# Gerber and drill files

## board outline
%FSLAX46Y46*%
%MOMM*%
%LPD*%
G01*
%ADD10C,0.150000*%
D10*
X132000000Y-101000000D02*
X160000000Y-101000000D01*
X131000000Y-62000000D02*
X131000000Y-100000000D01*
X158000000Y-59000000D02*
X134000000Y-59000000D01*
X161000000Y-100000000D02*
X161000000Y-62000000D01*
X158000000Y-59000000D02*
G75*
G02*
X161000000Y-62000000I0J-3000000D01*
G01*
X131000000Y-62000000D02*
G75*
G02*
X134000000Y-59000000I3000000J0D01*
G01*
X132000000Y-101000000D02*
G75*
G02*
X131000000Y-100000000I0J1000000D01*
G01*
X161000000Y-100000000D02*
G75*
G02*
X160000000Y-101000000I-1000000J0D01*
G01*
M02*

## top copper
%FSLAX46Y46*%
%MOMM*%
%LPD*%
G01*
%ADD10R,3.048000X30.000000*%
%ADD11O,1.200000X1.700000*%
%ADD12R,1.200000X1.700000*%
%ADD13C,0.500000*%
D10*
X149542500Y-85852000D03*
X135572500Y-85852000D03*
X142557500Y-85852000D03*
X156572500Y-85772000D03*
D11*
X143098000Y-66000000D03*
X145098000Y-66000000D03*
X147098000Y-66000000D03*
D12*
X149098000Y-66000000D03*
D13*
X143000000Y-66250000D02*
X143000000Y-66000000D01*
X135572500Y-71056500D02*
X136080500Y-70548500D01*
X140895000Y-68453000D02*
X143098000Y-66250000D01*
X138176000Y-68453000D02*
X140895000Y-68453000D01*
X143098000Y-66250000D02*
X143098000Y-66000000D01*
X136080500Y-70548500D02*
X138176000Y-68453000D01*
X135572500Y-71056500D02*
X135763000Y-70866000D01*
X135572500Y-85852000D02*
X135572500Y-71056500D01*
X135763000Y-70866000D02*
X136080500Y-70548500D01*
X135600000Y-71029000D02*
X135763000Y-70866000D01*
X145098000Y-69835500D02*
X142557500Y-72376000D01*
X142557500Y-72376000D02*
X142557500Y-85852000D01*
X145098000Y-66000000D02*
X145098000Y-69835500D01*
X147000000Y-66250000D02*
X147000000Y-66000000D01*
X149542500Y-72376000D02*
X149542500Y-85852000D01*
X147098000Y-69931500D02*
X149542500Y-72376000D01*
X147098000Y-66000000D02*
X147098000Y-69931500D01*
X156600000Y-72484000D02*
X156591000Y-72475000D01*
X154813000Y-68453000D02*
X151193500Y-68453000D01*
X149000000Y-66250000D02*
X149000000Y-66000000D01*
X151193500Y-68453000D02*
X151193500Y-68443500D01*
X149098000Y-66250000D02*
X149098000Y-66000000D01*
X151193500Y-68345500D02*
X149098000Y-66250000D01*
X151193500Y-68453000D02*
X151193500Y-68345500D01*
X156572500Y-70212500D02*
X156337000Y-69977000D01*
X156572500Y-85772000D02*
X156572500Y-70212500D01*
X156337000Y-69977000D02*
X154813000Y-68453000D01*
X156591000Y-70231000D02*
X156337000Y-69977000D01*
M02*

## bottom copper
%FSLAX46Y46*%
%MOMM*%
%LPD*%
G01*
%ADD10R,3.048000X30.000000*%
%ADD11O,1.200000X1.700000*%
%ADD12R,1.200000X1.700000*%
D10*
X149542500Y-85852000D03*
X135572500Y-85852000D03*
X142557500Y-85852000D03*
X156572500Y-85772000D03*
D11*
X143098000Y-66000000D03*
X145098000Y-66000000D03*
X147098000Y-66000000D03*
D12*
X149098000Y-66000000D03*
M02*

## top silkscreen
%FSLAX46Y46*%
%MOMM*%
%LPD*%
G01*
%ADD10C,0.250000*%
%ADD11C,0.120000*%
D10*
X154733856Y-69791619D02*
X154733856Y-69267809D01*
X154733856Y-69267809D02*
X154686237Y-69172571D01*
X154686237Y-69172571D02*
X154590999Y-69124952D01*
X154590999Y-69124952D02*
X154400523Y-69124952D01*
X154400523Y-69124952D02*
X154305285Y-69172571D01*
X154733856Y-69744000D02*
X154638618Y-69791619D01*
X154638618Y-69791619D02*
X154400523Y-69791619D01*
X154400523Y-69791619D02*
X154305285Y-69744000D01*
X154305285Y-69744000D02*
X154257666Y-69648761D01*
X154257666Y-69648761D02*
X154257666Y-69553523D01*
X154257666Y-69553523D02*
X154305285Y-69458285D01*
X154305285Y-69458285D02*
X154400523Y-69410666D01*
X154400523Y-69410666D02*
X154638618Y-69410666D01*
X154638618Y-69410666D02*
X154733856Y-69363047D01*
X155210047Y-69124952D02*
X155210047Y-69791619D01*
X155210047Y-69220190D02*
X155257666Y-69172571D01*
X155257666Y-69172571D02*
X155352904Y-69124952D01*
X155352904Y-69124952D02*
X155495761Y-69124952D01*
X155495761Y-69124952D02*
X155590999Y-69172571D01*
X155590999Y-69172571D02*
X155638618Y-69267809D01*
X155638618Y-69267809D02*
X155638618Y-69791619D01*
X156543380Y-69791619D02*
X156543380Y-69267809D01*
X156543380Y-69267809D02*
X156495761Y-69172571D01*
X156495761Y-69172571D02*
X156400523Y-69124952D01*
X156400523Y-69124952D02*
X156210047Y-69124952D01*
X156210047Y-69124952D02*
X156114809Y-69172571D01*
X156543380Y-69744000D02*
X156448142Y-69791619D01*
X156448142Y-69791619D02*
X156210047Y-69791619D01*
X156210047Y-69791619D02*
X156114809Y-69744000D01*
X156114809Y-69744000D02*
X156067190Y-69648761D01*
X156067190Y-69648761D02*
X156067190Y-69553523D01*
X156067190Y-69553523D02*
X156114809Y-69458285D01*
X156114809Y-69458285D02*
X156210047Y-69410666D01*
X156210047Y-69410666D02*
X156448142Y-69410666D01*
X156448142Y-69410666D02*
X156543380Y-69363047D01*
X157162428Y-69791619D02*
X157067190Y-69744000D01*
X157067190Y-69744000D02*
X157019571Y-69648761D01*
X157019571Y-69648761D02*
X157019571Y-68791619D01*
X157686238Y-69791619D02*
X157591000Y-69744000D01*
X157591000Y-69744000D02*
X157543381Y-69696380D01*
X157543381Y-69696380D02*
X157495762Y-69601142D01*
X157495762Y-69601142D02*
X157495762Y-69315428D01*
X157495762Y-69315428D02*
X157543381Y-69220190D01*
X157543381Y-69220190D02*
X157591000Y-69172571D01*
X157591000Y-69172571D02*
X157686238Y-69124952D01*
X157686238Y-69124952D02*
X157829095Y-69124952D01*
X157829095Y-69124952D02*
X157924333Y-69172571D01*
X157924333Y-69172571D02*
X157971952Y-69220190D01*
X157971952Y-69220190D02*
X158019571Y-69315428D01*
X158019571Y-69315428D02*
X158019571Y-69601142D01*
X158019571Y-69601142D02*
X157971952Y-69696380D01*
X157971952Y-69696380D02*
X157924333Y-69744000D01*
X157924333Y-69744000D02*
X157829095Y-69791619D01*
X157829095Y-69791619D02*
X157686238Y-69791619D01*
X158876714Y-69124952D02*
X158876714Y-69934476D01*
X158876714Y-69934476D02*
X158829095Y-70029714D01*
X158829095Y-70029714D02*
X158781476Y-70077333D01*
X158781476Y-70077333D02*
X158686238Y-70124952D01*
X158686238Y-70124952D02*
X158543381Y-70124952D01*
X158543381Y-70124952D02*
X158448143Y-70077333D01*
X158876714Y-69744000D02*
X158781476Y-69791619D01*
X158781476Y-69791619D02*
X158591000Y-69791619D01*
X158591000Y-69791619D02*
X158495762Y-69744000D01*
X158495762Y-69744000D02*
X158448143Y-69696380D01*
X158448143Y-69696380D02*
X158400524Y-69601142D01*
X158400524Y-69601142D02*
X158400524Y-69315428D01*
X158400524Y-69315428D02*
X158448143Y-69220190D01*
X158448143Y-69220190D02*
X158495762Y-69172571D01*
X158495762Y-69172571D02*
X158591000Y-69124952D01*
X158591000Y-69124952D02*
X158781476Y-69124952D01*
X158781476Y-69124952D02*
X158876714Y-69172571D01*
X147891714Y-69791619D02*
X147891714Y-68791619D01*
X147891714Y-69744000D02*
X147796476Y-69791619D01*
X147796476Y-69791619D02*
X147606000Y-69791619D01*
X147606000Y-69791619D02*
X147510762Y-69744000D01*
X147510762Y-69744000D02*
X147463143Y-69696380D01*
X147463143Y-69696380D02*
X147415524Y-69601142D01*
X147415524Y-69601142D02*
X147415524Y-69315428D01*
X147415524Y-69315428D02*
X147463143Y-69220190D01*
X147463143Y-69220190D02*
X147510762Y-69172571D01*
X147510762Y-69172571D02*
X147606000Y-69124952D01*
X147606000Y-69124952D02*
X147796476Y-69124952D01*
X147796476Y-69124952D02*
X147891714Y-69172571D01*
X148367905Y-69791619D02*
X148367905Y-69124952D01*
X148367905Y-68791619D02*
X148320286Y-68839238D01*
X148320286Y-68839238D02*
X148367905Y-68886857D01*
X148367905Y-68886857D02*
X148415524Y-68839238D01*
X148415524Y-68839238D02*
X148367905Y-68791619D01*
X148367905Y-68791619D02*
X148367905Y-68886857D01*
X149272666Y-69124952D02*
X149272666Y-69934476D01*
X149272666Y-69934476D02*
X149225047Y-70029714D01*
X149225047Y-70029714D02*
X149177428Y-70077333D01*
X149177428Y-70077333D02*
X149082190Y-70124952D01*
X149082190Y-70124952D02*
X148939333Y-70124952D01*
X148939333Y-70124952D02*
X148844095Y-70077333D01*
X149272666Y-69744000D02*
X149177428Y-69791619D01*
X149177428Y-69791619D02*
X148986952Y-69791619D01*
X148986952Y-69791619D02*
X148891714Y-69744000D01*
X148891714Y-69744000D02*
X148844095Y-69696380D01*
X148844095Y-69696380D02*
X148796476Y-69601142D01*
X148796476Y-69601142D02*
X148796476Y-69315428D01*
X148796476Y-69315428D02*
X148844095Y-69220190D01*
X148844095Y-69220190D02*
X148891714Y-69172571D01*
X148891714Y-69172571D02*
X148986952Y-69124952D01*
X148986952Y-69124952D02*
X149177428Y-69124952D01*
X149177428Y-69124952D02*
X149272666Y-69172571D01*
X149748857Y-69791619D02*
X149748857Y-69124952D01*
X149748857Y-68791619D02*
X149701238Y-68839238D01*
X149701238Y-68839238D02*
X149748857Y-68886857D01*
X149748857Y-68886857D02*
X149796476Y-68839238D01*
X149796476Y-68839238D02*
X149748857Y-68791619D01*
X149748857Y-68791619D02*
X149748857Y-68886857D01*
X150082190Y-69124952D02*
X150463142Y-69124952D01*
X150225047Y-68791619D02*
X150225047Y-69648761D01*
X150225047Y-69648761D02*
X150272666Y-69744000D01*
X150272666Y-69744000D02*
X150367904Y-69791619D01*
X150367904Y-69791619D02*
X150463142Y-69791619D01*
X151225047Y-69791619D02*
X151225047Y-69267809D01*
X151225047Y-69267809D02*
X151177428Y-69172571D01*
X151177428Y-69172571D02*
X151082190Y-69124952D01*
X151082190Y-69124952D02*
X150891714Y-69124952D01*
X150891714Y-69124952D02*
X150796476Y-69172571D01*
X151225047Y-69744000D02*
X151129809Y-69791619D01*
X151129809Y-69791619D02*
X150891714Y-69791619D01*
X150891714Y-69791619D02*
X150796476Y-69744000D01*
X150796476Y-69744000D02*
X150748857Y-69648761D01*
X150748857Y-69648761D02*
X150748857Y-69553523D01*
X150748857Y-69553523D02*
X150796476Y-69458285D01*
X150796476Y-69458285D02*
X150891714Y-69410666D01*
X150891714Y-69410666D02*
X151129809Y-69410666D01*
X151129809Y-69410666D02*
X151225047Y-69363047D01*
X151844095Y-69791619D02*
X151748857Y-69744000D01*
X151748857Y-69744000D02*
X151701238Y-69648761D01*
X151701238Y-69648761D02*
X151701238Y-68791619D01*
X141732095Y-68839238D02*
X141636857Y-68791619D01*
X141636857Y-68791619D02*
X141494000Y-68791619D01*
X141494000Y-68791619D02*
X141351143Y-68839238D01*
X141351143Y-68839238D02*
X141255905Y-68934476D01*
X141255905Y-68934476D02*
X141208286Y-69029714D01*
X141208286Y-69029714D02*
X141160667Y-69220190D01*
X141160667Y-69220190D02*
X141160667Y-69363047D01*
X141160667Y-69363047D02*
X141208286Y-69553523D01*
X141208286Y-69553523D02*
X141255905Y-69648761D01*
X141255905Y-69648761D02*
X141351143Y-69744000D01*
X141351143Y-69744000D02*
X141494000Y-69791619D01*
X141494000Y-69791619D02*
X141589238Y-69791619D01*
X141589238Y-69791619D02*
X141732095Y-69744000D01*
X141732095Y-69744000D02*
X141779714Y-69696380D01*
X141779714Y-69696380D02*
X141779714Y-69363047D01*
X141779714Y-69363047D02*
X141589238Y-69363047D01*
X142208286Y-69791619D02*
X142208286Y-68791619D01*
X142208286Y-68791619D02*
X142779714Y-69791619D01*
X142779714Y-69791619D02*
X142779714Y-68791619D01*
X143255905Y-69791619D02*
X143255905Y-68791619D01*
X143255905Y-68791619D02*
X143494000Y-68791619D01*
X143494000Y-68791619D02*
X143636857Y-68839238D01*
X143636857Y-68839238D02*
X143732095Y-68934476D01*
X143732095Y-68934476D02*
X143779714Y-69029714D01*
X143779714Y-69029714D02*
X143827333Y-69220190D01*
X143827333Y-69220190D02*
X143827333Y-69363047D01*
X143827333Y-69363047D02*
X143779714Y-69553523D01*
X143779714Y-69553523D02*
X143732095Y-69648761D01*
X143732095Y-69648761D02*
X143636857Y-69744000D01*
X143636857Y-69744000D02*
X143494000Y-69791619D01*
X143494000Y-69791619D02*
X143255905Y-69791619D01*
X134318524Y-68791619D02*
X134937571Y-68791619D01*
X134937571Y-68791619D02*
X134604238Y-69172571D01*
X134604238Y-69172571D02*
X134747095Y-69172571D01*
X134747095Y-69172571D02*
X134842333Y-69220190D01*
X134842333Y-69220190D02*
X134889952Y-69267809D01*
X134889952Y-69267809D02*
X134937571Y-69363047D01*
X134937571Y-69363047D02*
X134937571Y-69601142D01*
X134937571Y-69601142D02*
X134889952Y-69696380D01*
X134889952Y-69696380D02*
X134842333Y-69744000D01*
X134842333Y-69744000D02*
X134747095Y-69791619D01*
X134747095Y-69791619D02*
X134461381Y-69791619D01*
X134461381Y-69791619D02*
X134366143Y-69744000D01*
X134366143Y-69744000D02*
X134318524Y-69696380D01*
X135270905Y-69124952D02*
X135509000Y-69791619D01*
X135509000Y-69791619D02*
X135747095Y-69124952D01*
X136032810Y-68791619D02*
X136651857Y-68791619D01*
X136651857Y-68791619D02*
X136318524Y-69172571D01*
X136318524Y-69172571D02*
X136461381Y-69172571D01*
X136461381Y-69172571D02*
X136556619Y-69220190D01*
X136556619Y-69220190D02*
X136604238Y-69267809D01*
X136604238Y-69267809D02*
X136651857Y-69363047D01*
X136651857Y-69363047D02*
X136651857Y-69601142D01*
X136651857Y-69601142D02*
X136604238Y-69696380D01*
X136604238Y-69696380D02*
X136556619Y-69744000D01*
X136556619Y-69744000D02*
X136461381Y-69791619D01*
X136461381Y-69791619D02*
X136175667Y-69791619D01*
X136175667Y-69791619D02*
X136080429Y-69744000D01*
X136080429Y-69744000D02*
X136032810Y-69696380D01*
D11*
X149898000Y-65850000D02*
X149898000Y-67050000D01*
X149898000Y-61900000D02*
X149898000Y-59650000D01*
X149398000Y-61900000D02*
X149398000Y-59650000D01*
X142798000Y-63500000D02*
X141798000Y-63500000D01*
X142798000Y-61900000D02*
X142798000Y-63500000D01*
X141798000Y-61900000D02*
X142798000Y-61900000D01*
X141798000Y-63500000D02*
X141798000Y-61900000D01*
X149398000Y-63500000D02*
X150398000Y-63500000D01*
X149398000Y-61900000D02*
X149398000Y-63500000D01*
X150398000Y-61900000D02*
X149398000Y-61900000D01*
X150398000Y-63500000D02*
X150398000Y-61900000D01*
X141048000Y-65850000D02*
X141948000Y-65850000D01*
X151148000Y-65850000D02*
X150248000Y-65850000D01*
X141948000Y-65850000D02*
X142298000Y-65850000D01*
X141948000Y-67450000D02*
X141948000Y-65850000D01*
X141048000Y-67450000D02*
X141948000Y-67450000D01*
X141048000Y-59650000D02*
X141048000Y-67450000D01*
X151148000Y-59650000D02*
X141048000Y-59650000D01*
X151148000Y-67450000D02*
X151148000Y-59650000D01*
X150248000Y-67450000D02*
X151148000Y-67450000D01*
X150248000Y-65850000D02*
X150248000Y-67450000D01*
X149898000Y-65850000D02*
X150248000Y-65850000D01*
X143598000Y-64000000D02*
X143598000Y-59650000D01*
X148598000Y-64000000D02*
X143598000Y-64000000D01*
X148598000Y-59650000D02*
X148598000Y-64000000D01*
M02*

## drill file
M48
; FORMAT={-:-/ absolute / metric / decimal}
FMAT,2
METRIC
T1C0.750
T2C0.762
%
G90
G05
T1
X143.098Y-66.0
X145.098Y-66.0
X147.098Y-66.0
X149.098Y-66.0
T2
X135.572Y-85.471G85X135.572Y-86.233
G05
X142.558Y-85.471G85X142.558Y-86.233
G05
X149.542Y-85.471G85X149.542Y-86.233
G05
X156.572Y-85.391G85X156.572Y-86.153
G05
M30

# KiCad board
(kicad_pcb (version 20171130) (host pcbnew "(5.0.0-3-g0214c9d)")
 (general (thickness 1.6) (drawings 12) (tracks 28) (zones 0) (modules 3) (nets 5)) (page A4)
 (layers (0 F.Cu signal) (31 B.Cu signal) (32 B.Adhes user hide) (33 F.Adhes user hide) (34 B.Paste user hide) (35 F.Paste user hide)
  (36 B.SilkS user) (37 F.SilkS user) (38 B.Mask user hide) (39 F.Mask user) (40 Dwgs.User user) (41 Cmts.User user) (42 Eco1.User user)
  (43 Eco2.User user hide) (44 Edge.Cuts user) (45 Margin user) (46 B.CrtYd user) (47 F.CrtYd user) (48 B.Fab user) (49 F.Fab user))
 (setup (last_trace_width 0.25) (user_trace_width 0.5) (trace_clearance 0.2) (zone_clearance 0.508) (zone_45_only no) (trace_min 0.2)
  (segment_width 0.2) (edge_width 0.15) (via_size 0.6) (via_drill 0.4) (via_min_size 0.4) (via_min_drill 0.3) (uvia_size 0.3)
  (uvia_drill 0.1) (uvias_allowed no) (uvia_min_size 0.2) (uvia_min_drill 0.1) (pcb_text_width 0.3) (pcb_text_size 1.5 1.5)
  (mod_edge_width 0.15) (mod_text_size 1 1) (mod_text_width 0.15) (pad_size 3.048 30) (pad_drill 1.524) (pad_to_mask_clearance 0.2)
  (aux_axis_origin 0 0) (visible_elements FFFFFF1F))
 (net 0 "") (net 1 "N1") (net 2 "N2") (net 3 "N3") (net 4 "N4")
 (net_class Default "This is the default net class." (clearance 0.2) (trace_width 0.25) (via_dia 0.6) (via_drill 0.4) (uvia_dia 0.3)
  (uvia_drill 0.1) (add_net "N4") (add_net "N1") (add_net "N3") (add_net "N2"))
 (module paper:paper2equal (layer B.Cu) (at 145.7325 70.612)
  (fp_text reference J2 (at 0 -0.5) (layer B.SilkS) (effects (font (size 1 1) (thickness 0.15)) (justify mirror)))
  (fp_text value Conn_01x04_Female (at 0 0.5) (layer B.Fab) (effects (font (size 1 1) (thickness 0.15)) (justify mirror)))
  (pad 3 thru_hole rect (at 3.81 15.24) (size 3.048 30) (drill oval 0.762 1.524) (layers *.Cu *.Mask) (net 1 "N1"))
  (pad 1 thru_hole rect (at -10.16 15.24) (size 3.048 30) (drill oval 0.762 1.524) (layers *.Cu *.Mask) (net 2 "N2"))
  (pad 2 thru_hole rect (at -3.175 15.24) (size 3.048 30) (drill oval 0.762 1.524) (layers *.Cu *.Mask) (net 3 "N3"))
  (pad 4 thru_hole rect (at 10.84 15.16) (size 3.048 30) (drill oval 0.762 1.524) (layers *.Cu *.Mask) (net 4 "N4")))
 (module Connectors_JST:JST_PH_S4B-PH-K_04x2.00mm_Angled (layer F.Cu) (at 149.098 66 180)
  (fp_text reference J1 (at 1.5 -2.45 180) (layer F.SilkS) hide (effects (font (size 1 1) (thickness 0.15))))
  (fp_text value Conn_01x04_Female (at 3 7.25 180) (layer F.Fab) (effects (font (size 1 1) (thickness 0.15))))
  (fp_line (start -0.8 0.15) (end -0.8 -1.05) (layer F.SilkS) (width 0.12))
  (fp_line (start -0.8 4.1) (end -0.8 6.35) (layer F.SilkS) (width 0.12))
  (fp_line (start -0.3 4.1) (end -0.3 6.35) (layer F.SilkS) (width 0.12))
  (fp_line (start 6.3 2.5) (end 7.3 2.5) (layer F.SilkS) (width 0.12))
  (fp_line (start 6.3 4.1) (end 6.3 2.5) (layer F.SilkS) (width 0.12))
  (fp_line (start 7.3 4.1) (end 6.3 4.1) (layer F.SilkS) (width 0.12))
  (fp_line (start 7.3 2.5) (end 7.3 4.1) (layer F.SilkS) (width 0.12))
  (fp_line (start -0.3 2.5) (end -1.3 2.5) (layer F.SilkS) (width 0.12))
  (fp_line (start -0.3 4.1) (end -0.3 2.5) (layer F.SilkS) (width 0.12))
  (fp_line (start -1.3 4.1) (end -0.3 4.1) (layer F.SilkS) (width 0.12))
  (fp_line (start -1.3 2.5) (end -1.3 4.1) (layer F.SilkS) (width 0.12))
  (fp_line (start 8.05 0.15) (end 7.15 0.15) (layer F.SilkS) (width 0.12))
  (fp_line (start -2.05 0.15) (end -1.15 0.15) (layer F.SilkS) (width 0.12))
  (fp_line (start 7.15 0.15) (end 6.8 0.15) (layer F.SilkS) (width 0.12))
  (fp_line (start 7.15 -1.45) (end 7.15 0.15) (layer F.SilkS) (width 0.12))
  (fp_line (start 8.05 -1.45) (end 7.15 -1.45) (layer F.SilkS) (width 0.12))
  (fp_line (start 8.05 6.35) (end 8.05 -1.45) (layer F.SilkS) (width 0.12))
  (fp_line (start -2.05 6.35) (end 8.05 6.35) (layer F.SilkS) (width 0.12))
  (fp_line (start -2.05 -1.45) (end -2.05 6.35) (layer F.SilkS) (width 0.12))
  (fp_line (start -1.15 -1.45) (end -2.05 -1.45) (layer F.SilkS) (width 0.12))
  (fp_line (start -1.15 0.15) (end -1.15 -1.45) (layer F.SilkS) (width 0.12))
  (fp_line (start -0.8 0.15) (end -1.15 0.15) (layer F.SilkS) (width 0.12))
  (fp_line (start 5.5 2) (end 5.5 6.35) (layer F.SilkS) (width 0.12))
  (fp_line (start 0.5 2) (end 5.5 2) (layer F.SilkS) (width 0.12))
  (fp_line (start 0.5 6.35) (end 0.5 2) (layer F.SilkS) (width 0.12))
  (pad 4 thru_hole oval (at 6 0 180) (size 1.2 1.7) (drill 0.75) (layers *.Cu *.Mask) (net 2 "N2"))
  (pad 3 thru_hole oval (at 4 0 180) (size 1.2 1.7) (drill 0.75) (layers *.Cu *.Mask) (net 3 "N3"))
  (pad 2 thru_hole oval (at 2 0 180) (size 1.2 1.7) (drill 0.75) (layers *.Cu *.Mask) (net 1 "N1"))
  (pad 1 thru_hole rect (at 0 0 180) (size 1.2 1.7) (drill 0.75) (layers *.Cu *.Mask) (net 4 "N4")))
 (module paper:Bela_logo (layer B.Cu) (at 155.067 64.897 135)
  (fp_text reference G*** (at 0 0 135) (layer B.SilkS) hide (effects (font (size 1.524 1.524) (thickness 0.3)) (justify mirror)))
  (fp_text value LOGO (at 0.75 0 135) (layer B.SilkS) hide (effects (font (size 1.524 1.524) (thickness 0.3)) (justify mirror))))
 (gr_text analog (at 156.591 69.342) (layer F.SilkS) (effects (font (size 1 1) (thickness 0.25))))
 (gr_line (start 132 101) (end 160 101) (angle 90) (layer Edge.Cuts) (width 0.15))
 (gr_line (start 131 62) (end 131 100) (angle 90) (layer Edge.Cuts) (width 0.15))
 (gr_line (start 158 59) (end 134 59) (angle 90) (layer Edge.Cuts) (width 0.15))
 (gr_line (start 161 100) (end 161 62) (angle 90) (layer Edge.Cuts) (width 0.15))
 (gr_arc (start 158 62) (end 158 59) (angle 90) (layer Edge.Cuts) (width 0.15))
 (gr_arc (start 134 62) (end 131 62) (angle 90) (layer Edge.Cuts) (width 0.15))
 (gr_arc (start 132 100) (end 132 101) (angle 90) (layer Edge.Cuts) (width 0.15))
 (gr_arc (start 160 100) (end 161 100) (angle 90) (layer Edge.Cuts) (width 0.15))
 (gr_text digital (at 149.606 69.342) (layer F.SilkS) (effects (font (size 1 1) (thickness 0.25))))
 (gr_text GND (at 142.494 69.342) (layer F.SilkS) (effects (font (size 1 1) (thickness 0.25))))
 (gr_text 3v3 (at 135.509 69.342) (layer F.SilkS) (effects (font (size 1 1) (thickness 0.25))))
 (segment (start 143 66.25) (end 143 66) (width 0.5) (layer F.Cu) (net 2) (status 30))
 (segment (start 135.5725 71.0565) (end 136.0805 70.5485) (width 0.5) (layer F.Cu) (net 2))
 (segment (start 140.895 68.453) (end 143.098 66.25) (width 0.5) (layer F.Cu) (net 2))
 (segment (start 138.176 68.453) (end 140.895 68.453) (width 0.5) (layer F.Cu) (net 2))
 (segment (start 143.098 66.25) (end 143.098 66) (width 0.5) (layer F.Cu) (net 2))
 (segment (start 136.0805 70.5485) (end 138.176 68.453) (width 0.5) (layer F.Cu) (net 2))
 (segment (start 135.5725 71.0565) (end 135.763 70.866) (width 0.5) (layer F.Cu) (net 2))
 (segment (start 135.5725 85.852) (end 135.5725 71.0565) (width 0.5) (layer F.Cu) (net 2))
 (segment (start 135.763 70.866) (end 136.0805 70.5485) (width 0.5) (layer F.Cu) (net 2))
 (segment (start 135.6 71.029) (end 135.763 70.866) (width 0.5) (layer F.Cu) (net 2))
 (segment (start 145.098 69.8355) (end 142.5575 72.376) (width 0.5) (layer F.Cu) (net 3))
 (segment (start 142.5575 72.376) (end 142.5575 85.852) (width 0.5) (layer F.Cu) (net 3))
 (segment (start 145.098 66) (end 145.098 69.8355) (width 0.5) (layer F.Cu) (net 3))
 (segment (start 147 66.25) (end 147 66) (width 0.5) (layer F.Cu) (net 1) (status 30))
 (segment (start 149.5425 72.376) (end 149.5425 85.852) (width 0.5) (layer F.Cu) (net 1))
 (segment (start 147.098 69.9315) (end 149.5425 72.376) (width 0.5) (layer F.Cu) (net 1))
 (segment (start 147.098 66) (end 147.098 69.9315) (width 0.5) (layer F.Cu) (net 1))
 (segment (start 156.6 72.484) (end 156.591 72.475) (width 0.5) (layer F.Cu) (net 4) (status 30))
 (segment (start 154.813 68.453) (end 151.1935 68.453) (width 0.5) (layer F.Cu) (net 4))
 (segment (start 149 66.25) (end 149 66) (width 0.5) (layer F.Cu) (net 4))
 (segment (start 151.1935 68.453) (end 151.1935 68.4435) (width 0.5) (layer F.Cu) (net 4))
 (segment (start 149.098 66.25) (end 149.098 66) (width 0.5) (layer F.Cu) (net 4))
 (segment (start 151.1935 68.3455) (end 149.098 66.25) (width 0.5) (layer F.Cu) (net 4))
 (segment (start 151.1935 68.453) (end 151.1935 68.3455) (width 0.5) (layer F.Cu) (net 4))
 (segment (start 156.5725 70.2125) (end 156.337 69.977) (width 0.5) (layer F.Cu) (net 4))
 (segment (start 156.5725 85.772) (end 156.5725 70.2125) (width 0.5) (layer F.Cu) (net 4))
 (segment (start 156.337 69.977) (end 154.813 68.453) (width 0.5) (layer F.Cu) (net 4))
 (segment (start 156.591 70.231) (end 156.337 69.977) (width 0.5) (layer F.Cu) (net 4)))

